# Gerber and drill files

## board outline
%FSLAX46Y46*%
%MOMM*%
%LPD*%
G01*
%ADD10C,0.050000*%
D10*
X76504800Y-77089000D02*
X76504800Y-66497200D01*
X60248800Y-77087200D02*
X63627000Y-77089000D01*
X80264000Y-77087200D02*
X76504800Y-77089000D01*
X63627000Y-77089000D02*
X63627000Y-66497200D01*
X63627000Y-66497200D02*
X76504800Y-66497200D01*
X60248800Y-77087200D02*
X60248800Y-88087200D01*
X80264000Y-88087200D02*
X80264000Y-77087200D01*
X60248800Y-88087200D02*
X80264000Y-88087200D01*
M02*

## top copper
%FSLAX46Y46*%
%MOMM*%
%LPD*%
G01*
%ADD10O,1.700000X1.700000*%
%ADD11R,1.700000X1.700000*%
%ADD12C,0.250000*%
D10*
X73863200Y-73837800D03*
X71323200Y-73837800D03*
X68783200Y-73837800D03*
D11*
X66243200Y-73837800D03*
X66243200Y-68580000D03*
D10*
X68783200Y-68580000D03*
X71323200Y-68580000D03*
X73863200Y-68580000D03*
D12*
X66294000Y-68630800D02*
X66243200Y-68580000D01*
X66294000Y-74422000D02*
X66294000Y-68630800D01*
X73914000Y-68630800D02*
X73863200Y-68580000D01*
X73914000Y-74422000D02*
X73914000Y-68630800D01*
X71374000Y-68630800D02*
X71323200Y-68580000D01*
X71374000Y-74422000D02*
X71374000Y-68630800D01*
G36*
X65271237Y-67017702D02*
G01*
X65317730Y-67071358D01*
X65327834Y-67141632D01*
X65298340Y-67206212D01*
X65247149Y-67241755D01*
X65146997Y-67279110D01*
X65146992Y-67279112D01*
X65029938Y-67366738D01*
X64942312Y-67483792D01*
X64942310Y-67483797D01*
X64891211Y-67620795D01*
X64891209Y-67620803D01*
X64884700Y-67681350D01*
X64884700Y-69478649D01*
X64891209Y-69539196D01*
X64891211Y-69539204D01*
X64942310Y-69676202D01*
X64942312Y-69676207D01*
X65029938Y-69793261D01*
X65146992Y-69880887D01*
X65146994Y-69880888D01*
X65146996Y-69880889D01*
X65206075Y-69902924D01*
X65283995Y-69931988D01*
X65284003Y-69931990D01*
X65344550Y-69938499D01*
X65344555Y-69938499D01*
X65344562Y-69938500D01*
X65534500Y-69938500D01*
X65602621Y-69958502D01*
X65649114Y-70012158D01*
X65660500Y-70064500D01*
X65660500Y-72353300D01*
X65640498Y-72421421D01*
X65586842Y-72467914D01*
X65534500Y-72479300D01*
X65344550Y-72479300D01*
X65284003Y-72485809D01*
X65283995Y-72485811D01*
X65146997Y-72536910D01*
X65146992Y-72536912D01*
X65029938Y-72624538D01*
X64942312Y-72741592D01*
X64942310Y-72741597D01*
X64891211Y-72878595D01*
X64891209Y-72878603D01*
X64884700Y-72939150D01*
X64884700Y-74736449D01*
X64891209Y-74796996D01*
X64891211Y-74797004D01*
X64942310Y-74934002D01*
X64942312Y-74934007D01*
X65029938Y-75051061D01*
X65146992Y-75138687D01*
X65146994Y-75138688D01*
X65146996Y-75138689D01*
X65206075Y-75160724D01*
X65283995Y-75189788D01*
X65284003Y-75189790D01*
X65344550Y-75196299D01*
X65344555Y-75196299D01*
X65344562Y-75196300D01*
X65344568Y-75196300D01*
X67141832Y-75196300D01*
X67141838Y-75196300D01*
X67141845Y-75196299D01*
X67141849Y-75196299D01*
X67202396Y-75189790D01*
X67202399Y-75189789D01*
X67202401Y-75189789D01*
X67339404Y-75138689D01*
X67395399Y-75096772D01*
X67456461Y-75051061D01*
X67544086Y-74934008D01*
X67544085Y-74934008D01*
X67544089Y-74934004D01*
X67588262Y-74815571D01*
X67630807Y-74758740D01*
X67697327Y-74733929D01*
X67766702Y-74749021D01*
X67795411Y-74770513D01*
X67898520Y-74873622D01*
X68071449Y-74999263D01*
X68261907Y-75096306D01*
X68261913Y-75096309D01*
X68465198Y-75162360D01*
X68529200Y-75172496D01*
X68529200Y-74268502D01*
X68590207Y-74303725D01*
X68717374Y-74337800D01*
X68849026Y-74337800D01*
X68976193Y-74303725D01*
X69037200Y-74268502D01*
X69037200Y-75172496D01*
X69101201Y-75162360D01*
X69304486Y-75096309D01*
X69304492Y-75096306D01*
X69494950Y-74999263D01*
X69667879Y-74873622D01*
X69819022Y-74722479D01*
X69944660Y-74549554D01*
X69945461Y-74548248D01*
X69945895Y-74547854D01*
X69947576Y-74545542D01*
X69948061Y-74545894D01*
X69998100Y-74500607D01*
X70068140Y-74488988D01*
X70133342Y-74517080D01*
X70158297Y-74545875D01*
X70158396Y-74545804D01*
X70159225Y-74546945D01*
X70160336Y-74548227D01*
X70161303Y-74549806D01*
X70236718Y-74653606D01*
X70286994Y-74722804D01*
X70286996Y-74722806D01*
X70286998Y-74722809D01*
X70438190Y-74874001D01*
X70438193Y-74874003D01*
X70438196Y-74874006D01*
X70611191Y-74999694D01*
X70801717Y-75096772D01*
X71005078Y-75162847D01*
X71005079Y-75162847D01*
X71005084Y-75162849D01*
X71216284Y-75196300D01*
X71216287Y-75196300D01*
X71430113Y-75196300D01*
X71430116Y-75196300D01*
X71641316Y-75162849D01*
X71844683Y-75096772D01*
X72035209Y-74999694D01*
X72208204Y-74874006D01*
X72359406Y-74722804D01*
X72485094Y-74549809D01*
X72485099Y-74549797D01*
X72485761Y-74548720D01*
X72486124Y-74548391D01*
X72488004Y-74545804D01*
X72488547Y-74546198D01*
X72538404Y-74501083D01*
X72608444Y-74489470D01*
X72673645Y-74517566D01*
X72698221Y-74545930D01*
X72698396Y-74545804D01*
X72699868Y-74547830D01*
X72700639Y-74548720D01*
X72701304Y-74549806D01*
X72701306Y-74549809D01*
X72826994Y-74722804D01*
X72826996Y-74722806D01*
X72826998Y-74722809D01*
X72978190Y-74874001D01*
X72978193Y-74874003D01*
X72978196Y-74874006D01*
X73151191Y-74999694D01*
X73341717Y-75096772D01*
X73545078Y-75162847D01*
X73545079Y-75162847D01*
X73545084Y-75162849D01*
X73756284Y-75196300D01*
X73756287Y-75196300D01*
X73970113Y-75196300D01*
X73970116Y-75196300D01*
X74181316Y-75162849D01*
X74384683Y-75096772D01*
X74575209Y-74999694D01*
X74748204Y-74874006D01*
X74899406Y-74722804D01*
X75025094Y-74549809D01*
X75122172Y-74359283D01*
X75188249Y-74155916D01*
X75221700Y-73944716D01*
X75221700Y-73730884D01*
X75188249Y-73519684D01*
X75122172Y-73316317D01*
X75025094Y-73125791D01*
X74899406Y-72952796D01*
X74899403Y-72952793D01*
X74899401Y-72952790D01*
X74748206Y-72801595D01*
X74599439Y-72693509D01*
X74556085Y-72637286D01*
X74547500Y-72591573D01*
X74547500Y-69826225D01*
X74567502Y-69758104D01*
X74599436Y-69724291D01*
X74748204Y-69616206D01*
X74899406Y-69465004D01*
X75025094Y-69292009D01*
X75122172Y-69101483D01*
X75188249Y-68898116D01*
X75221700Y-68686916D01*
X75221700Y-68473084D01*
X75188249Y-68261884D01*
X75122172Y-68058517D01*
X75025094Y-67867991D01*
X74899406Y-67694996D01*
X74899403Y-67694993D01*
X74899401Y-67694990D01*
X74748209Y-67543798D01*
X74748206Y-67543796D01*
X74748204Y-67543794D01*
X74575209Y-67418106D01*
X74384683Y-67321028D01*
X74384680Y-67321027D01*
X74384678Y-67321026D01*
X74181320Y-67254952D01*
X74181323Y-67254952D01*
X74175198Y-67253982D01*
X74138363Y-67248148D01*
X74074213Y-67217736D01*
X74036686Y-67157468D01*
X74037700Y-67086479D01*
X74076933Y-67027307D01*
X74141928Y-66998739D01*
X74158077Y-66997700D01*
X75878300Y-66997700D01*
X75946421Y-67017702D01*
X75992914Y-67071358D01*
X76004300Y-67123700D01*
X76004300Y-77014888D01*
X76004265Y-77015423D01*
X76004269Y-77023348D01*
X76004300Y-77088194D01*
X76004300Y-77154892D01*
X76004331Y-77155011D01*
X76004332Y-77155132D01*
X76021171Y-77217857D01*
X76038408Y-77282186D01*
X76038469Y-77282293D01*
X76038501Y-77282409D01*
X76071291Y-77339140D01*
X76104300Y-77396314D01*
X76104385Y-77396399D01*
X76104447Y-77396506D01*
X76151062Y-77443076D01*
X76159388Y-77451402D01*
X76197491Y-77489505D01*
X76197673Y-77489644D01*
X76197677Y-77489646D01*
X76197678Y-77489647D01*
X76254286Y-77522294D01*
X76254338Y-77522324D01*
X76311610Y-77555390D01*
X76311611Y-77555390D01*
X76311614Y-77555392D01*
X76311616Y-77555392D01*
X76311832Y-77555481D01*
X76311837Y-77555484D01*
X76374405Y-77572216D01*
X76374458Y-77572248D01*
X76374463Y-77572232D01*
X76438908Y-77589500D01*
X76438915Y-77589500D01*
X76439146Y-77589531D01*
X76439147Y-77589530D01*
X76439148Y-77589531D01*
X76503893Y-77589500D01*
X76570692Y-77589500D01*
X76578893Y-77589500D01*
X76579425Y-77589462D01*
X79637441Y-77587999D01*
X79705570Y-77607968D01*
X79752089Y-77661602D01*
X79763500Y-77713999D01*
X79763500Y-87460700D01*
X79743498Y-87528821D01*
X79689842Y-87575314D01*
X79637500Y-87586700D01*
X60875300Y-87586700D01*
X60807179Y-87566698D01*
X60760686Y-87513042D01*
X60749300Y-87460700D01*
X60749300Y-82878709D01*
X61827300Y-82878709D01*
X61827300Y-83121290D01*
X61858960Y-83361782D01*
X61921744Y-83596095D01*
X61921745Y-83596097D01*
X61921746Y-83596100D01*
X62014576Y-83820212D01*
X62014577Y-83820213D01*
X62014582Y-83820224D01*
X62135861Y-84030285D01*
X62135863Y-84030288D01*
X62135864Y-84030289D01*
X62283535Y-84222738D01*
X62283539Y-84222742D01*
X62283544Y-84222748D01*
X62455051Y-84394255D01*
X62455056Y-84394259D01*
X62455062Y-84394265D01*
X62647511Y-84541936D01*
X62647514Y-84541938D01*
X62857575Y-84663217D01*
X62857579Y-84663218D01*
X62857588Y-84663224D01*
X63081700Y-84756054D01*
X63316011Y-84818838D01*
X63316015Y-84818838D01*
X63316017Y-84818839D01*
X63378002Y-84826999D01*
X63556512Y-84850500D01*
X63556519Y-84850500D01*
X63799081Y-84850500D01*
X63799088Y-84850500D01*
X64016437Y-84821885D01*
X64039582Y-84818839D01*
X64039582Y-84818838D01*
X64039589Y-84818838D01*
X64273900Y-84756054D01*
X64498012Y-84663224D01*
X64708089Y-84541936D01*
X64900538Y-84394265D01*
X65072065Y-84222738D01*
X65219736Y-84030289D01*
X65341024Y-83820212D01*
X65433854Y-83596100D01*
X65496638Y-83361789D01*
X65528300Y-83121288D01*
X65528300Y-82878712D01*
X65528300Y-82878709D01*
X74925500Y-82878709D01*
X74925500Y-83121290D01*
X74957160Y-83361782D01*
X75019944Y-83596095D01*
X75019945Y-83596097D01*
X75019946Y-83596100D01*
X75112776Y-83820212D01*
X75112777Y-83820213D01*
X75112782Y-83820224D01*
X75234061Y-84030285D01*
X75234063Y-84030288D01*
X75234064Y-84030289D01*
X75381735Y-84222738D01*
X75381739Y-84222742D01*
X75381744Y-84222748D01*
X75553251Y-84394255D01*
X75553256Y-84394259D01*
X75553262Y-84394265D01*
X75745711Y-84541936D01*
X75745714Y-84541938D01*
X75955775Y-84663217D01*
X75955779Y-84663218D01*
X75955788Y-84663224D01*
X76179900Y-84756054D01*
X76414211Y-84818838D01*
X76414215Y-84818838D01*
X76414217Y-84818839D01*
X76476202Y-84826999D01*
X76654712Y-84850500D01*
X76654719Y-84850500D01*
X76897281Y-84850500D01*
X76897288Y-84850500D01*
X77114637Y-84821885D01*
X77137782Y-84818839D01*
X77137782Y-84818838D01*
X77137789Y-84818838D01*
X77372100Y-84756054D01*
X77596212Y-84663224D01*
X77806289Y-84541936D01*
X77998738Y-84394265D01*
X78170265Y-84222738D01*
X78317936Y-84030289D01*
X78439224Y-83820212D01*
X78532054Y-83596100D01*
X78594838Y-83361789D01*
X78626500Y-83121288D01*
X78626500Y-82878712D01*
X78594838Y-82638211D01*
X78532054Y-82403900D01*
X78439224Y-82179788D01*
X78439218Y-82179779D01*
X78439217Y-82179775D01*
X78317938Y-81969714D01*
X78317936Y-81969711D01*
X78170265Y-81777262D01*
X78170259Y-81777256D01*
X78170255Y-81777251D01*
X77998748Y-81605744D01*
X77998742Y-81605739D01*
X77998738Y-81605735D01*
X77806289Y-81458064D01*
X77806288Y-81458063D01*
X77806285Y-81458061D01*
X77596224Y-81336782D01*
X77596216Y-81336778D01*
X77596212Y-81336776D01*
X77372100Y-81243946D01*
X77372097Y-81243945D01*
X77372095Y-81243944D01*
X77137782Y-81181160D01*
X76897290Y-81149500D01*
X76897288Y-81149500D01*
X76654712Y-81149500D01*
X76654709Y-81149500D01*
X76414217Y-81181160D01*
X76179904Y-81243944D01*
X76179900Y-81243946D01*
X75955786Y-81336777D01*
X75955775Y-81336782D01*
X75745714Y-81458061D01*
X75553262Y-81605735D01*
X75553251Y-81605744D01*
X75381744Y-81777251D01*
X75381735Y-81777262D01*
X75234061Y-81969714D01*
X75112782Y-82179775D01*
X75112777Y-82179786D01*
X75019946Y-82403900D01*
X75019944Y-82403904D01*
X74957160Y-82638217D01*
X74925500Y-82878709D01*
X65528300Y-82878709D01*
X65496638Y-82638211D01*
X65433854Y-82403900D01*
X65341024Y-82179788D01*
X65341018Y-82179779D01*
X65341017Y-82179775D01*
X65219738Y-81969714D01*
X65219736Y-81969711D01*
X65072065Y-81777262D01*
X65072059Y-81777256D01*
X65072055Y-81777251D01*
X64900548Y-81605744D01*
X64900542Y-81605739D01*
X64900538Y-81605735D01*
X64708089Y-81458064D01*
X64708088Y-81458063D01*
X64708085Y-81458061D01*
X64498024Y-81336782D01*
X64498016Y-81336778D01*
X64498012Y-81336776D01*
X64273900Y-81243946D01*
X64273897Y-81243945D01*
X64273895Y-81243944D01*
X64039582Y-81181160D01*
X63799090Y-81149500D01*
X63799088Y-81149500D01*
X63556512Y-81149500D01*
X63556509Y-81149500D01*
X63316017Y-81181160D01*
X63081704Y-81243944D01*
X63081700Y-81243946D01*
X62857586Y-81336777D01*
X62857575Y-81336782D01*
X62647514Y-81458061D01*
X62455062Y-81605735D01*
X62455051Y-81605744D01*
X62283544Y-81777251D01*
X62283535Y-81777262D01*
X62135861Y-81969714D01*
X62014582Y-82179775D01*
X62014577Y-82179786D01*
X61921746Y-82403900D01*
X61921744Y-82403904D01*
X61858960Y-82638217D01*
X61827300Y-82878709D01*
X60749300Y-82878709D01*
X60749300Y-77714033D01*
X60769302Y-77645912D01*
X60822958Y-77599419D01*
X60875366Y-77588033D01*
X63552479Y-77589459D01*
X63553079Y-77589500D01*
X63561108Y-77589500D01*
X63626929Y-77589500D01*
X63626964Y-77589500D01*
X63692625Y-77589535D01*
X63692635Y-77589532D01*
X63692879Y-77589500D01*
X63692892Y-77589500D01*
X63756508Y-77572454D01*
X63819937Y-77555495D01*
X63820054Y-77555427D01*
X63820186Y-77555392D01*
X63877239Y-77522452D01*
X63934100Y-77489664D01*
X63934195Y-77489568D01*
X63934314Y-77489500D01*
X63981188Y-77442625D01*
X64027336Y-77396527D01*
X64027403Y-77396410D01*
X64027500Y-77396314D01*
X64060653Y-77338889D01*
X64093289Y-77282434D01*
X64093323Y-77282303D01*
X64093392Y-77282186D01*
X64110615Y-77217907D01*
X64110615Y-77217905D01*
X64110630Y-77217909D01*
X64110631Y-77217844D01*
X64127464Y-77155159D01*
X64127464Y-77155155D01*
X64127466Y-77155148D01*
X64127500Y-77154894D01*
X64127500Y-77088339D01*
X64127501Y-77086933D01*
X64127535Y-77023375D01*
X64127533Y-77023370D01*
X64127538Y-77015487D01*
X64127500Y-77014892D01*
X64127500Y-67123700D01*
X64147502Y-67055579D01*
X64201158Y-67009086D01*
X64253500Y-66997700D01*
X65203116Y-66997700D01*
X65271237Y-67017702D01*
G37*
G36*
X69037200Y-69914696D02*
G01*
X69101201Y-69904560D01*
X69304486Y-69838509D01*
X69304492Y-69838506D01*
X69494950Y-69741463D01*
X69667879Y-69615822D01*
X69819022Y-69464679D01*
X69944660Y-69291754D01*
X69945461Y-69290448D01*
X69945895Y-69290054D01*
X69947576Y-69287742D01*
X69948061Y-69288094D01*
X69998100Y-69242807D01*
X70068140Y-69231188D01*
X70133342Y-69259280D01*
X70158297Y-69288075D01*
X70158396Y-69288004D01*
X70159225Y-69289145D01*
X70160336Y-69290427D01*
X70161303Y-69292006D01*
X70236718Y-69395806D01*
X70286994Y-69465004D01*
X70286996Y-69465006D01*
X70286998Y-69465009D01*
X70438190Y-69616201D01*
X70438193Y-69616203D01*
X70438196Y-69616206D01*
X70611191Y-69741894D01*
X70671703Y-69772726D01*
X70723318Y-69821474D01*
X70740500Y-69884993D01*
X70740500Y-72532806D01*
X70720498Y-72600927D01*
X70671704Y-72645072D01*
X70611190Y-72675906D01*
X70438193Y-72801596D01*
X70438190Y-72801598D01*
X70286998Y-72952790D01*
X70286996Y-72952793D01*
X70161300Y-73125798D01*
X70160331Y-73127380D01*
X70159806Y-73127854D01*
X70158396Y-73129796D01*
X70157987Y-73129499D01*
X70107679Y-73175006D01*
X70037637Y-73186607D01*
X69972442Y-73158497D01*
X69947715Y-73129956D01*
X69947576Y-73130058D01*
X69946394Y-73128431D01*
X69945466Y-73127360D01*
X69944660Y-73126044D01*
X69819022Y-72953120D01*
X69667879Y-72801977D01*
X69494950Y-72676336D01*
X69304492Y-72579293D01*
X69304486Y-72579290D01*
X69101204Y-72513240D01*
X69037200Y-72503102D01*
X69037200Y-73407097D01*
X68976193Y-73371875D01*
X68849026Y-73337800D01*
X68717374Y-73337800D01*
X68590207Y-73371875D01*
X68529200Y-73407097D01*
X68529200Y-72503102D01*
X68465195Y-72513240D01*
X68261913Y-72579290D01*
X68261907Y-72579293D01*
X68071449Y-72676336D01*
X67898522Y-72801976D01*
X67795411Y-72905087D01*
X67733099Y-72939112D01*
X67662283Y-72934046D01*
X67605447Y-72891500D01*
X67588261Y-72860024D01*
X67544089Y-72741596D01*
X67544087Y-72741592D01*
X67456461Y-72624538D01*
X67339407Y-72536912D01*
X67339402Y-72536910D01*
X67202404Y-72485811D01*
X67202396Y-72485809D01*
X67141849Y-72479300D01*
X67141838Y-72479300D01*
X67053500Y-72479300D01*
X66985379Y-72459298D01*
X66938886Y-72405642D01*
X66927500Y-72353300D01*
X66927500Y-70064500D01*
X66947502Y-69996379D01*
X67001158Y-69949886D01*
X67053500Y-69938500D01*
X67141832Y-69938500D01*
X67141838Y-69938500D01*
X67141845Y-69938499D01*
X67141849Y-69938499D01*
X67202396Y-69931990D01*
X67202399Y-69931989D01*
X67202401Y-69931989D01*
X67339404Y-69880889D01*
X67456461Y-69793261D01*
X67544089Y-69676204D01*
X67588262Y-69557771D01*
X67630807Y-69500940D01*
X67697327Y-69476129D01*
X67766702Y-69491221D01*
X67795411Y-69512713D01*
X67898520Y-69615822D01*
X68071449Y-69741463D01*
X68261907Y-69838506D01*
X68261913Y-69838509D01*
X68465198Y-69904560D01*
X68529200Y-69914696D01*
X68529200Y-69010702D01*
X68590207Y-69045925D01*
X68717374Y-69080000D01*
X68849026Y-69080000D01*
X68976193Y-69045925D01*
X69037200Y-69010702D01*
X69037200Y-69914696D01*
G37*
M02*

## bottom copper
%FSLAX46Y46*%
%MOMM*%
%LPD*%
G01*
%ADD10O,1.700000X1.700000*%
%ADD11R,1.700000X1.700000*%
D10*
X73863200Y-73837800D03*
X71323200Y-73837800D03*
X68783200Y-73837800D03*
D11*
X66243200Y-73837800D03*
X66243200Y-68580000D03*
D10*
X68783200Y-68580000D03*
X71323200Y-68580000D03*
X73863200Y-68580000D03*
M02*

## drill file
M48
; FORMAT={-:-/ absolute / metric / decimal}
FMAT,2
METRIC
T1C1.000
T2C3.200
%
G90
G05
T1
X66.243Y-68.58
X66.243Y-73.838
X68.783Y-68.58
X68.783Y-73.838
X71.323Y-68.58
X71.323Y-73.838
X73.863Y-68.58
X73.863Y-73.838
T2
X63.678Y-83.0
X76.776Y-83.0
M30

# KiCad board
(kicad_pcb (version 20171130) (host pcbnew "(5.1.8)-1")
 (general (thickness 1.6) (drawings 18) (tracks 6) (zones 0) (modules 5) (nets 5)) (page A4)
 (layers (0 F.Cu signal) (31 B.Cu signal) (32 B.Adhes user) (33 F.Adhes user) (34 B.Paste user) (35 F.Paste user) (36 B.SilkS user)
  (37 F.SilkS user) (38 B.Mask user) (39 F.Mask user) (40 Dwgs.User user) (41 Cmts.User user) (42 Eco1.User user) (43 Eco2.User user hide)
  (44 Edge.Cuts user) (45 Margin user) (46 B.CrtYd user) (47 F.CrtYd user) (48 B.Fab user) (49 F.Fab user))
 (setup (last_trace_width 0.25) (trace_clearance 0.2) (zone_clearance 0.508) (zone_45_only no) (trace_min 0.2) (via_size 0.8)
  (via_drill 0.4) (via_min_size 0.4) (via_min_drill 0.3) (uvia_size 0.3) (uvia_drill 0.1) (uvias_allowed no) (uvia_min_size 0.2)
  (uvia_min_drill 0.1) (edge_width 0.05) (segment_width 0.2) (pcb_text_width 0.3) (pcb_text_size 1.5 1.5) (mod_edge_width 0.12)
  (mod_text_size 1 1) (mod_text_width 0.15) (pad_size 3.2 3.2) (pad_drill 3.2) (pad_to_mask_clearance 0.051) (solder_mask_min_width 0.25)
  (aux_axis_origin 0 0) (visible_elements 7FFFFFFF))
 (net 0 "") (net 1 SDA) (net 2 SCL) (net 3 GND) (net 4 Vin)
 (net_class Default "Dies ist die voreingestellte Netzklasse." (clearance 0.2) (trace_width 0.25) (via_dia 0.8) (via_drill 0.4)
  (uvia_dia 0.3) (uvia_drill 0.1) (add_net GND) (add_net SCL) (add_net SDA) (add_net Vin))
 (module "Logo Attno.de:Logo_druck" (layer F.Cu) (at 70.0786 81.6356)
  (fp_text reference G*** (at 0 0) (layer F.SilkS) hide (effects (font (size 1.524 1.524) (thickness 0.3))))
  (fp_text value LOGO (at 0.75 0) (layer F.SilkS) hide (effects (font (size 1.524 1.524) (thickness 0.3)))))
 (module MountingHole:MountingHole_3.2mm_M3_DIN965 (layer F.Cu) (at 76.776 83)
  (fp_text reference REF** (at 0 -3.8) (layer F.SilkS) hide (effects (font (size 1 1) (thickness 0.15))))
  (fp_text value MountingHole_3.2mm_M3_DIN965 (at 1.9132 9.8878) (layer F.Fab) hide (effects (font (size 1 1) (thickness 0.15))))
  (pad 1 np_thru_hole circle (at 0 0) (size 3.2 3.2) (drill 3.2) (layers *.Cu *.Mask)))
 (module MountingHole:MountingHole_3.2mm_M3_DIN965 (layer F.Cu) (at 63.6778 83)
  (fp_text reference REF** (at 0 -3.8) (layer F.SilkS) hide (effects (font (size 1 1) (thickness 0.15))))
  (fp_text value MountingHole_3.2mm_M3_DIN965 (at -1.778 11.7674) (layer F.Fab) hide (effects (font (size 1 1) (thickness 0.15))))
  (pad 1 np_thru_hole circle (at 0 0) (size 3.2 3.2) (drill 3.2) (layers *.Cu *.Mask)))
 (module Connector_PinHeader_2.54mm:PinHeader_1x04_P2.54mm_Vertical (layer F.Cu) (at 66.2432 73.8378 90)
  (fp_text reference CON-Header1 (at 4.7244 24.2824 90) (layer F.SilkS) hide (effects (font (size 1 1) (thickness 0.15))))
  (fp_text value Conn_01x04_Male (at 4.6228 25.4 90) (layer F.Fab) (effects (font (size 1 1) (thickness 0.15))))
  (pad 4 thru_hole oval (at 0 7.62 90) (size 1.7 1.7) (drill 1) (layers *.Cu *.Mask) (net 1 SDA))
  (pad 3 thru_hole oval (at 0 5.08 90) (size 1.7 1.7) (drill 1) (layers *.Cu *.Mask) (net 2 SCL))
  (pad 2 thru_hole oval (at 0 2.54 90) (size 1.7 1.7) (drill 1) (layers *.Cu *.Mask) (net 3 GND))
  (pad 1 thru_hole rect (at 0 0 90) (size 1.7 1.7) (drill 1) (layers *.Cu *.Mask) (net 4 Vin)))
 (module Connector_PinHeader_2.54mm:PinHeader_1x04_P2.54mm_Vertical (layer F.Cu) (at 66.2432 68.58 90)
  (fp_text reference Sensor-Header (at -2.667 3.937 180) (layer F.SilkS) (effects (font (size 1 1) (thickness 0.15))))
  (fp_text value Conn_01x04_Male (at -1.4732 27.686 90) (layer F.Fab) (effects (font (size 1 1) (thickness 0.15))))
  (pad 1 thru_hole rect (at 0 0 90) (size 1.7 1.7) (drill 1) (layers *.Cu *.Mask) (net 4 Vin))
  (pad 2 thru_hole oval (at 0 2.54 90) (size 1.7 1.7) (drill 1) (layers *.Cu *.Mask) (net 3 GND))
  (pad 3 thru_hole oval (at 0 5.08 90) (size 1.7 1.7) (drill 1) (layers *.Cu *.Mask) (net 2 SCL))
  (pad 4 thru_hole oval (at 0 7.62 90) (size 1.7 1.7) (drill 1) (layers *.Cu *.Mask) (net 1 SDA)))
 (gr_line (start 76.5048 77.089) (end 76.5048 66.4972) (layer Edge.Cuts) (width 0.05))
 (gr_line (start 60.2488 77.0872) (end 63.627 77.089) (layer Edge.Cuts) (width 0.05))
 (gr_line (start 80.264 77.0872) (end 76.5048 77.089) (layer Edge.Cuts) (width 0.05))
 (gr_line (start 63.627 77.089) (end 63.627 66.4972) (layer Edge.Cuts) (width 0.05))
 (gr_line (start 63.627 66.4972) (end 76.5048 66.4972) (layer Edge.Cuts) (width 0.05))
 (gr_line (start 60.2488 77.0872) (end 60.2488 88.0872) (layer Edge.Cuts) (width 0.05))
 (gr_line (start 80.264 88.0872) (end 80.264 77.0872) (layer Edge.Cuts) (width 0.05))
 (gr_line (start 60.2488 88.0872) (end 80.264 88.0872) (layer Edge.Cuts) (width 0.05))
 (segment (start 66.294 68.6308) (end 66.2432 68.58) (width 0.25) (layer F.Cu) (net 4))
 (segment (start 66.294 74.422) (end 66.294 68.6308) (width 0.25) (layer F.Cu) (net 4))
 (segment (start 73.914 68.6308) (end 73.8632 68.58) (width 0.25) (layer F.Cu) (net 1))
 (segment (start 73.914 74.422) (end 73.914 68.6308) (width 0.25) (layer F.Cu) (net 1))
 (segment (start 71.374 68.6308) (end 71.3232 68.58) (width 0.25) (layer F.Cu) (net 2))
 (segment (start 71.374 74.422) (end 71.374 68.6308) (width 0.25) (layer F.Cu) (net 2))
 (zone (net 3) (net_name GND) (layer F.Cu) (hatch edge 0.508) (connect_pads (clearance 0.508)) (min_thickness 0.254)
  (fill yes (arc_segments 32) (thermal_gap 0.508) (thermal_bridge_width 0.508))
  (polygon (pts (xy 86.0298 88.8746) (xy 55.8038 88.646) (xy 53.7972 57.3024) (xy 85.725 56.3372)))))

